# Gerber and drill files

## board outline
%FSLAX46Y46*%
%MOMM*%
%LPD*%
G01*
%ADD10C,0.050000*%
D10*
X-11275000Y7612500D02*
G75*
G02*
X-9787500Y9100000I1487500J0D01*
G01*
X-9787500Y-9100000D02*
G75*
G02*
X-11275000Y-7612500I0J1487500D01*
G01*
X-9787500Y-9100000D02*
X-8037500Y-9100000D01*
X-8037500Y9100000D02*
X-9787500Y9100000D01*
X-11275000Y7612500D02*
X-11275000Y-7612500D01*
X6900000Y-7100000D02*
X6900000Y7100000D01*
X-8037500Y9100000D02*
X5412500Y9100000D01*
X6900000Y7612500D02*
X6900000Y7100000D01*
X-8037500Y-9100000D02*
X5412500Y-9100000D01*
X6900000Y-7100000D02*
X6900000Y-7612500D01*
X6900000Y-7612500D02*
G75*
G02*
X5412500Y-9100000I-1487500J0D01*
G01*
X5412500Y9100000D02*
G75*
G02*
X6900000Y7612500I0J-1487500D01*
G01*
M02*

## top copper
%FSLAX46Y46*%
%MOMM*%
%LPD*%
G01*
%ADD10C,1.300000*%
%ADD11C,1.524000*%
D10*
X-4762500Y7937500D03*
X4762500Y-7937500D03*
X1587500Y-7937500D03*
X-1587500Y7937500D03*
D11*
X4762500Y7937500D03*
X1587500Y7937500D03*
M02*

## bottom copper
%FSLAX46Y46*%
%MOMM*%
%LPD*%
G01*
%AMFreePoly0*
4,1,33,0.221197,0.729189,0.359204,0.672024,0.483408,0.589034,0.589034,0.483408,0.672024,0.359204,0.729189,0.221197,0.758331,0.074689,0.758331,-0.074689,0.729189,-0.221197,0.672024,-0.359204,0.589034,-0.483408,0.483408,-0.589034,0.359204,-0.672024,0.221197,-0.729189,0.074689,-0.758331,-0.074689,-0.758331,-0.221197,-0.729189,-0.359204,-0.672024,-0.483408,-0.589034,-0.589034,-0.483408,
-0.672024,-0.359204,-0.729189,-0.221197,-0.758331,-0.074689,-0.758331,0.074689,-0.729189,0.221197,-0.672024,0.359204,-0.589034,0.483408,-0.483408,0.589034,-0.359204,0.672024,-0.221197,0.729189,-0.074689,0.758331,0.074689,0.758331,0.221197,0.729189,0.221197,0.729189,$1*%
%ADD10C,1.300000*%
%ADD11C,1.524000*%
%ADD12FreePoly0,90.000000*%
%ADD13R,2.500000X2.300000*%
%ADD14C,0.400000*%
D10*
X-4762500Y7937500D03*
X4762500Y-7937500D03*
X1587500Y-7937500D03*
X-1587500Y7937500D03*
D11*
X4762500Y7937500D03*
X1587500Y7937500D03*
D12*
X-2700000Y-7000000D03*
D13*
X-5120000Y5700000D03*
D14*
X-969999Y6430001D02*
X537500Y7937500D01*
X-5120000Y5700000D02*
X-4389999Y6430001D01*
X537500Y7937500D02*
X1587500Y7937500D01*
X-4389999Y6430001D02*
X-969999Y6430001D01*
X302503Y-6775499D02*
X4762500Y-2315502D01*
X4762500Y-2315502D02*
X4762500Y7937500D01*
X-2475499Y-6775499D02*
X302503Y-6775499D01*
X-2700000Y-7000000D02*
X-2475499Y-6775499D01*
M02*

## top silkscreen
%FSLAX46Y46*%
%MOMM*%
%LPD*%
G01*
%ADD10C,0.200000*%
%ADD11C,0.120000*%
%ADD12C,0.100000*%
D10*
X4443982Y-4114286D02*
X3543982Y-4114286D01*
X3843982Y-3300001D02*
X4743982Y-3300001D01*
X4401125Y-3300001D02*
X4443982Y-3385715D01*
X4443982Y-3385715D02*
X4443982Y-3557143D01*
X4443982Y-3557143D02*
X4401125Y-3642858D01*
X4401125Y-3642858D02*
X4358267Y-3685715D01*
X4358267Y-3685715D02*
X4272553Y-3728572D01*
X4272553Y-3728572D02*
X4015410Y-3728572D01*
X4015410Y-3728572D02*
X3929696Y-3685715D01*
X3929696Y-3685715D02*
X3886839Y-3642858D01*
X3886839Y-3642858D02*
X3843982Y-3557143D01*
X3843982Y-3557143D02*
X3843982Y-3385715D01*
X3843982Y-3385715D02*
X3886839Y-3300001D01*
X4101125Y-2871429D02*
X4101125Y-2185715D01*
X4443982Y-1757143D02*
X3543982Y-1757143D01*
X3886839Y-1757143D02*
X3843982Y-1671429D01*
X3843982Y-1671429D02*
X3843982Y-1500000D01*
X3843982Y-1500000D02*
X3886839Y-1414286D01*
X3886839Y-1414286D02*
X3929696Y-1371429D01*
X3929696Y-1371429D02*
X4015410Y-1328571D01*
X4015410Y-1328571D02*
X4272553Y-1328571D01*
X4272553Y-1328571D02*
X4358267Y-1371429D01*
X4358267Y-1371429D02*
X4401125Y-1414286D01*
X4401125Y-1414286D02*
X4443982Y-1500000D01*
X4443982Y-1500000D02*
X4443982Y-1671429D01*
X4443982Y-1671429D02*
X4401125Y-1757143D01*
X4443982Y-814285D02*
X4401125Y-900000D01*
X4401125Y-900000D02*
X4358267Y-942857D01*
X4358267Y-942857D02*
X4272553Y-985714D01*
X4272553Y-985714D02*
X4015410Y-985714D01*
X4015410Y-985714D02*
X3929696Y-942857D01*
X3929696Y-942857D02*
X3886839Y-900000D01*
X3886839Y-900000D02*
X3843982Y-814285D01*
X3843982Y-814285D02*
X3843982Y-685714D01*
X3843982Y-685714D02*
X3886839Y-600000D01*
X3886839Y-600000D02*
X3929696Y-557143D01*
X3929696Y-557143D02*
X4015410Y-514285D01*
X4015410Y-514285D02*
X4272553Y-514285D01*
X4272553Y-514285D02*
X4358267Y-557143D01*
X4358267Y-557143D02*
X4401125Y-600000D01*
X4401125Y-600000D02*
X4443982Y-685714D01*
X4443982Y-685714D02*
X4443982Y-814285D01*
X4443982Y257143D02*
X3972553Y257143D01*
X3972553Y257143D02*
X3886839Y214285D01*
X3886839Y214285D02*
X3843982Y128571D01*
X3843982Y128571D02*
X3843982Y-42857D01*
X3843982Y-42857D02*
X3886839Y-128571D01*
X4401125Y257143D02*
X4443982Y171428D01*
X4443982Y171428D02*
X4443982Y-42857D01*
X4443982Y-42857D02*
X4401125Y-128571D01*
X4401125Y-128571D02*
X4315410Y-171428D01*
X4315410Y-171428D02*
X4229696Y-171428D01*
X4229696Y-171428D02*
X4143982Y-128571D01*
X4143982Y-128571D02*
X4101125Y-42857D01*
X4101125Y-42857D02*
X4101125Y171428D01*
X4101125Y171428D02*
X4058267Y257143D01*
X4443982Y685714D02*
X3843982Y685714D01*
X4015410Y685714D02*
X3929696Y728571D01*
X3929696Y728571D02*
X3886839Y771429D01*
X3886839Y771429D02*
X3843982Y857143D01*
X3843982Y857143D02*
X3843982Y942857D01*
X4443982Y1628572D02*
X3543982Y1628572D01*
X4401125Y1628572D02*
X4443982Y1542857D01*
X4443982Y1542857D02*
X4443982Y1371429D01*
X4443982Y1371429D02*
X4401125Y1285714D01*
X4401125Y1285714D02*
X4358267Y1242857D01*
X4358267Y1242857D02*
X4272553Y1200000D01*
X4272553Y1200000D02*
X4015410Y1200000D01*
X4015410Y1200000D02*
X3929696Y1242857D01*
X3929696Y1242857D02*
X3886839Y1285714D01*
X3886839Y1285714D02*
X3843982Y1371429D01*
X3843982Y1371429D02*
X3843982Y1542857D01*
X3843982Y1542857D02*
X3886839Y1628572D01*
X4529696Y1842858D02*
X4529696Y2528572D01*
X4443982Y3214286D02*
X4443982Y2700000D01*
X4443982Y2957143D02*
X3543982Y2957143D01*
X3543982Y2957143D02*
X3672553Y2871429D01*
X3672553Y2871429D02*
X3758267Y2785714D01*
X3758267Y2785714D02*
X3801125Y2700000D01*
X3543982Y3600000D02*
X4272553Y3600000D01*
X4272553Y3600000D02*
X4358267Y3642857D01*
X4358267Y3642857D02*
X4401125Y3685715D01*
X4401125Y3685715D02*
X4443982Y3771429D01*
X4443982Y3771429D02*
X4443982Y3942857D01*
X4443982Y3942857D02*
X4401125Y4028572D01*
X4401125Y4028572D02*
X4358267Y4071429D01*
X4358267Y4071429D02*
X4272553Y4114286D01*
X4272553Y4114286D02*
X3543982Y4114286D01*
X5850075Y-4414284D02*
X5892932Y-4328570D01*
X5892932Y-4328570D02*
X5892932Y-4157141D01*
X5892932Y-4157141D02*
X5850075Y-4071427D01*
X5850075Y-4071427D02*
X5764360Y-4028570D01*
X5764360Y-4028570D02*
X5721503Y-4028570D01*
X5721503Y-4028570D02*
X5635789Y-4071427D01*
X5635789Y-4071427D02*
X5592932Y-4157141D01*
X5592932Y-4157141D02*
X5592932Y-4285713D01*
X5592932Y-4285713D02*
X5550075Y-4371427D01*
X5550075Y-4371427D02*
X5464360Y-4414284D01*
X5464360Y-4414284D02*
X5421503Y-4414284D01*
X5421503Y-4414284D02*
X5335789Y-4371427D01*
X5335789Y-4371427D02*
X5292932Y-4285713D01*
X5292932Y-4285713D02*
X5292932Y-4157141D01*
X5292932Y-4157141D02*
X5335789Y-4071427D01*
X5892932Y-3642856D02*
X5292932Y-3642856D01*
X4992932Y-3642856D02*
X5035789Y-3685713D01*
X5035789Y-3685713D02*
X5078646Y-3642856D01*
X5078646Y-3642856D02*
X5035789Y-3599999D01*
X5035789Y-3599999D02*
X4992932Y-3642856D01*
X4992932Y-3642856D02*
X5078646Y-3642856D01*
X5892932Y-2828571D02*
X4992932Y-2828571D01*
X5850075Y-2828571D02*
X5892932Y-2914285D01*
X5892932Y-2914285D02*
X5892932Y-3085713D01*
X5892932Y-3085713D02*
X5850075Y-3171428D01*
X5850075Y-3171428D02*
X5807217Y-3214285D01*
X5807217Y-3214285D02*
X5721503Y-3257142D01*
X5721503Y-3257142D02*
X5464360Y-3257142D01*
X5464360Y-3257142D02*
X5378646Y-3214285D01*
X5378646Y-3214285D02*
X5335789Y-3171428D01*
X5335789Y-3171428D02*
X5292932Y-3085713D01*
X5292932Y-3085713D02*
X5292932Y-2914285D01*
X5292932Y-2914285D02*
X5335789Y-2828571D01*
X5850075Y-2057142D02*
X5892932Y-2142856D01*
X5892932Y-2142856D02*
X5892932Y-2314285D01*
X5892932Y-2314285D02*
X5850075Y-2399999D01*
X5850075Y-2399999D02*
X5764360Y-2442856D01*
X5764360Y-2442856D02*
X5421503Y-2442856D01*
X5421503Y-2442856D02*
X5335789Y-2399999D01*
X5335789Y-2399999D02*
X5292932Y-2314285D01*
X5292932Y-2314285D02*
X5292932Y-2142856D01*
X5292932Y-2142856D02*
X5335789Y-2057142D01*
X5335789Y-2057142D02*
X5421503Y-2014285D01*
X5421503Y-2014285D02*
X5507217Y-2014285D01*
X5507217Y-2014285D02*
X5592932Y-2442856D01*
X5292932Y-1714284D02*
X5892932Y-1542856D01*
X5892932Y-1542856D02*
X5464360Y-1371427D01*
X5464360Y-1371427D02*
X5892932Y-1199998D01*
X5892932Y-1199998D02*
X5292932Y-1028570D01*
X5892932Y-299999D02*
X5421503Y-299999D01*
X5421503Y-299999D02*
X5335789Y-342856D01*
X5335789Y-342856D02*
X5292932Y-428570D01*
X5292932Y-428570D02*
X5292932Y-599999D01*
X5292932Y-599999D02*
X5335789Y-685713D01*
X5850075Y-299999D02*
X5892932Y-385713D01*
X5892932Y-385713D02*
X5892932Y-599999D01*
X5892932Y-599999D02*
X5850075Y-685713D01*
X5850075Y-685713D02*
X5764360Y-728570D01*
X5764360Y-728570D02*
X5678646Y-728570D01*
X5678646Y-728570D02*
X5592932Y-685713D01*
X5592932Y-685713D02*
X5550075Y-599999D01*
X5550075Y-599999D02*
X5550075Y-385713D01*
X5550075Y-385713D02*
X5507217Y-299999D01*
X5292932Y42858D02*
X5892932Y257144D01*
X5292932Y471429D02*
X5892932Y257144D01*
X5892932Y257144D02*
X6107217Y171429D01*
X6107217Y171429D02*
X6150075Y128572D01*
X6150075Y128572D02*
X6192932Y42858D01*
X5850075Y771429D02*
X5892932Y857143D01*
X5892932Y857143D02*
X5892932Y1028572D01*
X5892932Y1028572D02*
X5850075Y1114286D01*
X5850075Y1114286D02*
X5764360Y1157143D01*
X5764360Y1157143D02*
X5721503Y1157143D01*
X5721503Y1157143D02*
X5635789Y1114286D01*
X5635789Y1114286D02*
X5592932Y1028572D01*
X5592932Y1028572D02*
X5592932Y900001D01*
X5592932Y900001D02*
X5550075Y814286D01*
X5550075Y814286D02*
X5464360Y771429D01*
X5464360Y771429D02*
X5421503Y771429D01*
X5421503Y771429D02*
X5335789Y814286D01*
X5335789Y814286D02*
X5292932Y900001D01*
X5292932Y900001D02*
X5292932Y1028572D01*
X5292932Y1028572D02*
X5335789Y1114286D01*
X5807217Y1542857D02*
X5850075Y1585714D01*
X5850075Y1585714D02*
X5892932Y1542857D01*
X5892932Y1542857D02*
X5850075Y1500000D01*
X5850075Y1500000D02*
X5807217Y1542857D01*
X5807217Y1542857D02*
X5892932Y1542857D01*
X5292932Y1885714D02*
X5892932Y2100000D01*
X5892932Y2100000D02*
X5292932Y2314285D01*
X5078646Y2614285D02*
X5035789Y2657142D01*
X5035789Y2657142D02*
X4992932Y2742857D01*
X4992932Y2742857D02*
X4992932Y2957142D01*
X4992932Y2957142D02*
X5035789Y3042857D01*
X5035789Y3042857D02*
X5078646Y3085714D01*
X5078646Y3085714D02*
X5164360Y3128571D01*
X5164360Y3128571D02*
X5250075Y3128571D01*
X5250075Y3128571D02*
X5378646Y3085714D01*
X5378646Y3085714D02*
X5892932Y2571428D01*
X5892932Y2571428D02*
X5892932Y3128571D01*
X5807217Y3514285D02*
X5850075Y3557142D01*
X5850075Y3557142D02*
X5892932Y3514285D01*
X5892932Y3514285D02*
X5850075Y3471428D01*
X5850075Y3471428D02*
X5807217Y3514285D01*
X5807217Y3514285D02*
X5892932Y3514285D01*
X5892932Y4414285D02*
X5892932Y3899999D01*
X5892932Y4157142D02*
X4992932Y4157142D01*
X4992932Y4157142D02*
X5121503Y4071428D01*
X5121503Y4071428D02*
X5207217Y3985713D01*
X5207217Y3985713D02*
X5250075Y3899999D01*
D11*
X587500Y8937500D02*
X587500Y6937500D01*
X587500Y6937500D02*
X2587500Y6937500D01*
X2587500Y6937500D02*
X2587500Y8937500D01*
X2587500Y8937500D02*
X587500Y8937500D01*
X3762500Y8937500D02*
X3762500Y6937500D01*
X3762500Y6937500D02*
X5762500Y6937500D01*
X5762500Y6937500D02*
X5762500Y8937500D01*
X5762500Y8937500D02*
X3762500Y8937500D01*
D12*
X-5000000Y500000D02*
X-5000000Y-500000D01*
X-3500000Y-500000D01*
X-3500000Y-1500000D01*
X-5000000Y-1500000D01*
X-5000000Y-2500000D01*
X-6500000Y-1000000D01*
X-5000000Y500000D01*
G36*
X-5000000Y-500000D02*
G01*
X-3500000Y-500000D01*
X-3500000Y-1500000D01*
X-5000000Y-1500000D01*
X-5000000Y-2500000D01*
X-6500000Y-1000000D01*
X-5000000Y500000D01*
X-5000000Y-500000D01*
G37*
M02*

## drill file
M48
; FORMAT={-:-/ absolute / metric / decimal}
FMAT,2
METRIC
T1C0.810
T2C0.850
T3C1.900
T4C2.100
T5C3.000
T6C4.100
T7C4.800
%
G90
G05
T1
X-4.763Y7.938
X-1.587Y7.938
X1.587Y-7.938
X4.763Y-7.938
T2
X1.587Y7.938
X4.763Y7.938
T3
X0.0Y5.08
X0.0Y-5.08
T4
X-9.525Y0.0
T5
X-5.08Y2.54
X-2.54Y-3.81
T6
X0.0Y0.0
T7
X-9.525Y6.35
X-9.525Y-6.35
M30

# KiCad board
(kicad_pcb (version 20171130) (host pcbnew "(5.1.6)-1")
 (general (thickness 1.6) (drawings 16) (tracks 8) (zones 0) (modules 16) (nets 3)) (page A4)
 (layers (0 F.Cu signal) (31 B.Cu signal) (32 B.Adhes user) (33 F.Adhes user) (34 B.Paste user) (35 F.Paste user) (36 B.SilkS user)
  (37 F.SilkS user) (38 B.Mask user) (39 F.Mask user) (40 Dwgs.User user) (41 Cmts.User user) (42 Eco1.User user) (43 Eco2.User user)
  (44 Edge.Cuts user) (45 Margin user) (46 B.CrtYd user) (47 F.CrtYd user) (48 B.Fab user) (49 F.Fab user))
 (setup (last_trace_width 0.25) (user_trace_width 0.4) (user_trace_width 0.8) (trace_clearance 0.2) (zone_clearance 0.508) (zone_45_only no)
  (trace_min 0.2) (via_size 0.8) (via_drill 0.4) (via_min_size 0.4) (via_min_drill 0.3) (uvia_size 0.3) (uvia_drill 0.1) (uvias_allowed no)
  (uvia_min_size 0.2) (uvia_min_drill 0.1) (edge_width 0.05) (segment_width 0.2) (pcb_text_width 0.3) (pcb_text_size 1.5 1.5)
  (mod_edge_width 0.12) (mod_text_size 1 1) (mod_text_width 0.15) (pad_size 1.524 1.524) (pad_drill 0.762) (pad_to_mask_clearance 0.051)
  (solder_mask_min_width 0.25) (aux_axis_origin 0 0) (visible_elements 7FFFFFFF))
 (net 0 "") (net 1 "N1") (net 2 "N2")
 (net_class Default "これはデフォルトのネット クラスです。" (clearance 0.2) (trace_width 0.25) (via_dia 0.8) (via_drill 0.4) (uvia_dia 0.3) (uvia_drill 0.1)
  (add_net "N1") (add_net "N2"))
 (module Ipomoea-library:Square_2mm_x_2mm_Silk (layer F.Cu) (at 1.5875 -7.9375)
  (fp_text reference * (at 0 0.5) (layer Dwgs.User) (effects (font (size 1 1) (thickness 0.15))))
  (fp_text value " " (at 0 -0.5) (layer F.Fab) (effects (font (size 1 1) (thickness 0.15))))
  (fp_line (start -1 -1) (end -1 1) (layer F.SilkS) (width 0.12))
  (fp_line (start -1 1) (end 1 1) (layer F.SilkS) (width 0.12))
  (fp_line (start 1 1) (end 1 -1) (layer F.SilkS) (width 0.12))
  (fp_line (start 1 -1) (end -1 -1) (layer F.SilkS) (width 0.12)))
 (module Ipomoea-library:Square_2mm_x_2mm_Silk (layer F.Cu) (at 4.7625 -7.9375)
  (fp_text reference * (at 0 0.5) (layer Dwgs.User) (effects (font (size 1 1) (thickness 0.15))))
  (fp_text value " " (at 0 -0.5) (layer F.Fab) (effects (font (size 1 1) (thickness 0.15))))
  (fp_line (start -1 -1) (end -1 1) (layer F.SilkS) (width 0.12))
  (fp_line (start -1 1) (end 1 1) (layer F.SilkS) (width 0.12))
  (fp_line (start 1 1) (end 1 -1) (layer F.SilkS) (width 0.12))
  (fp_line (start 1 -1) (end -1 -1) (layer F.SilkS) (width 0.12)))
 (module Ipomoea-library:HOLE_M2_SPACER (layer F.Cu) (at -9.525 6.35)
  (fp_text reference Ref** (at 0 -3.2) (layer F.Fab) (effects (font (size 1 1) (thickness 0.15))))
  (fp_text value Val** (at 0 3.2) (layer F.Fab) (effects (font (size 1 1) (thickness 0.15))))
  (pad "" np_thru_hole circle (at 0 0) (size 4.8 4.8) (drill 4.8) (layers *.Cu *.Mask)))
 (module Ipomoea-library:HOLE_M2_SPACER (layer F.Cu) (at -9.525 -6.35)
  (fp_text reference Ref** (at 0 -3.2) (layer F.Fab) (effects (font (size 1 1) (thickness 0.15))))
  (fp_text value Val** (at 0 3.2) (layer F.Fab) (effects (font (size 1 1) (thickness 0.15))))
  (pad "" np_thru_hole circle (at 0 0) (size 4.8 4.8) (drill 4.8) (layers *.Cu *.Mask)))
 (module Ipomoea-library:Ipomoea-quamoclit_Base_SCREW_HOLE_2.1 (layer F.Cu) (at -9.525 0)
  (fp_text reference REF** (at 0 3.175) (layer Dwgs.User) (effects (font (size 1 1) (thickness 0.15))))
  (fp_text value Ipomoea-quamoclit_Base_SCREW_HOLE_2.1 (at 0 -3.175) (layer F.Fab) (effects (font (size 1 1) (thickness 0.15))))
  (pad "" np_thru_hole circle (at 0 0) (size 2.1 2.1) (drill 2.1) (layers *.Cu *.Mask)))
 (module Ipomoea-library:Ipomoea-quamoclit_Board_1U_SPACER (layer F.Cu) (at 0 0)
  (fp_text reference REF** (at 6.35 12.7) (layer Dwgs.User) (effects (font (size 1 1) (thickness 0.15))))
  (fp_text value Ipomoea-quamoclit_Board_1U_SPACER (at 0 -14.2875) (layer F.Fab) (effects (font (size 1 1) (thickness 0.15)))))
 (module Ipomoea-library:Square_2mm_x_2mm (layer F.Cu) (at 1.5875 7.9375)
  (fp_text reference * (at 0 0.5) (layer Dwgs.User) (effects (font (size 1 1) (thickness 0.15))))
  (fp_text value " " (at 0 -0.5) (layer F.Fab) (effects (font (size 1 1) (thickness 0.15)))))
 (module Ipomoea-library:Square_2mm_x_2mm (layer F.Cu) (at 4.7625 7.9375)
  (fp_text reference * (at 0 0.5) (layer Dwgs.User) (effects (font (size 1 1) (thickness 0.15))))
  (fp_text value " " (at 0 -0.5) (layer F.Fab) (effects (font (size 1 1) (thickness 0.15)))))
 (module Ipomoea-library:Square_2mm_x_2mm (layer F.Cu) (at -4.7625 -7.9375)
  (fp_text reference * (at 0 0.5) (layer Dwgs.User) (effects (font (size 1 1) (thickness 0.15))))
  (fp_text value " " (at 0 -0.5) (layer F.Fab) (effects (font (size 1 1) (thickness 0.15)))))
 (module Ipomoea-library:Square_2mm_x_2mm (layer F.Cu) (at -1.5875 -7.9375)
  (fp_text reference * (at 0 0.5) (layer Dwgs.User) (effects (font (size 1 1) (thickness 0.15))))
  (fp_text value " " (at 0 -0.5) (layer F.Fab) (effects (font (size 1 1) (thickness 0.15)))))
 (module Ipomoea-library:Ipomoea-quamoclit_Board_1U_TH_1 (layer F.Cu) (at -4.7625 -7.9375)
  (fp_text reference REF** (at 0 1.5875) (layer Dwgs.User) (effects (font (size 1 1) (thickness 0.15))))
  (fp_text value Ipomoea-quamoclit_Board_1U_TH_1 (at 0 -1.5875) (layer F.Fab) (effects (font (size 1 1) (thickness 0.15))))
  (pad "" thru_hole circle (at 0 0 180) (size 1.3 1.3) (drill 0.81) (layers *.Cu *.Mask)))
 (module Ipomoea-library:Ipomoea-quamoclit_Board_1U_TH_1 (layer F.Cu) (at 4.7625 7.9375)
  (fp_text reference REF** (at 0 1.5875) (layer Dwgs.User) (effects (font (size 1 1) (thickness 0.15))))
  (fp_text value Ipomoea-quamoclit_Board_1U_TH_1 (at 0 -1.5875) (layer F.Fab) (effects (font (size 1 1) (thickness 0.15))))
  (pad "" thru_hole circle (at 0 0 180) (size 1.3 1.3) (drill 0.81) (layers *.Cu *.Mask)))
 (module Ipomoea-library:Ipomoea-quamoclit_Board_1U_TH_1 (layer F.Cu) (at 1.5875 7.9375)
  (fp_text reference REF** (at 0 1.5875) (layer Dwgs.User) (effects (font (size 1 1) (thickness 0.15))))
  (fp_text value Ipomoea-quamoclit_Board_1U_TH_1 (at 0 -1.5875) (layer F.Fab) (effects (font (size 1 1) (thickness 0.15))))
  (pad "" thru_hole circle (at 0 0 180) (size 1.3 1.3) (drill 0.81) (layers *.Cu *.Mask)))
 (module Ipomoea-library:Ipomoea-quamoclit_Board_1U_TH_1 (layer F.Cu) (at -1.5875 -7.9375)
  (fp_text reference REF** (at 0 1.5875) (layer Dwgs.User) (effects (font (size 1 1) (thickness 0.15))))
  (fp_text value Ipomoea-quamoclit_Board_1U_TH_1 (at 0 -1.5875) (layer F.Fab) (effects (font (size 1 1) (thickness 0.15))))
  (pad "" thru_hole circle (at 0 0 180) (size 1.3 1.3) (drill 0.81) (layers *.Cu *.Mask)))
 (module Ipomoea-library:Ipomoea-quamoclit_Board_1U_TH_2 (layer F.Cu) (at 3.175 -7.9375 180)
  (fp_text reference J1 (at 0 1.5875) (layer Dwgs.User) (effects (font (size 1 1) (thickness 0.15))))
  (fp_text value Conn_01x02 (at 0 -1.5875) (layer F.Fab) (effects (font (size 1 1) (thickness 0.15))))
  (pad 1 thru_hole circle (at -1.5875 0) (size 1.524 1.524) (drill 0.85) (layers *.Cu *.Mask) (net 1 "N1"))
  (pad 2 thru_hole circle (at 1.5875 0) (size 1.524 1.524) (drill 0.85) (layers *.Cu *.Mask) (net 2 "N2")))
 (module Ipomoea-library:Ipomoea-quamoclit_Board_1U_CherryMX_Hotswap (layer F.Cu) (at 0 0 90)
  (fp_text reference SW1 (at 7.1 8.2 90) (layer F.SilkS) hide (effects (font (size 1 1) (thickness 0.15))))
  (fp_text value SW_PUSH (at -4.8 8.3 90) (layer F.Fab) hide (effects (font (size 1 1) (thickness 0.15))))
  (fp_poly (pts (xy 0.5 -5) (xy -0.5 -5) (xy -0.5 -3.5) (xy -1.5 -3.5) (xy -1.5 -5) (xy -2.5 -5) (xy -1 -6.5)) (layer F.SilkS) (width 0.1))
  (pad "" np_thru_hole circle (at 0 0 180) (size 4.1 4.1) (drill 4.1) (layers *.Cu *.Mask))
  (pad "" np_thru_hole circle (at 5.08 0 90) (size 1.9 1.9) (drill 1.9) (layers *.Cu *.Mask))
  (pad "" np_thru_hole circle (at -5.08 0 90) (size 1.9 1.9) (drill 1.9) (layers *.Cu *.Mask))
  (pad 1 smd custom (at -7 -2.7 90) (size 1.524 1.524) (layers B.Cu B.Paste B.Mask) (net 1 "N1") (zone_connect 0)
   (options (clearance outline) (anchor circle)) (primitives))
  (pad "" np_thru_hole circle (at 2.54 -5.08 270) (size 3 3) (drill 3) (layers *.Cu *.Mask))
  (pad 2 smd rect (at 5.7 -5.12 270) (size 2.3 2.5) (layers B.Cu B.Paste B.Mask) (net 2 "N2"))
  (pad "" np_thru_hole circle (at -3.81 -2.54 270) (size 3 3) (drill 3) (layers *.Cu *.Mask)))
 (gr_arc (start -9.7875 -7.6125) (end -9.7875 -9.1) (angle -90) (layer Edge.Cuts) (width 0.05))
 (gr_arc (start -9.7875 7.6125) (end -11.275 7.6125) (angle -90) (layer Edge.Cuts) (width 0.05))
 (gr_line (start -9.7875 9.1) (end -8.0375 9.1) (layer Edge.Cuts) (width 0.05))
 (gr_line (start -8.0375 -9.1) (end -9.7875 -9.1) (layer Edge.Cuts) (width 0.05))
 (gr_line (start -11.275 -7.6125) (end -11.275 7.6125) (layer Edge.Cuts) (width 0.05))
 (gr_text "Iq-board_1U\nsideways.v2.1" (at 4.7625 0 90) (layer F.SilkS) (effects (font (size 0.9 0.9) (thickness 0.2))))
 (gr_line (start 6.9 7.1) (end 6.9 -7.1) (layer Edge.Cuts) (width 0.05))
 (gr_line (start -8.0375 -9.1) (end 5.4125 -9.1) (layer Edge.Cuts) (width 0.05))
 (gr_line (start 6.9 -7.6125) (end 6.9 -7.1) (layer Edge.Cuts) (width 0.05))
 (gr_line (start -8.0375 9.1) (end 5.4125 9.1) (layer Edge.Cuts) (width 0.05))
 (gr_line (start 6.9 7.1) (end 6.9 7.6125) (layer Edge.Cuts) (width 0.05))
 (gr_arc (start 5.4125 7.6125) (end 5.4125 9.1) (angle -90) (layer Edge.Cuts) (width 0.05))
 (gr_arc (start 5.4125 -7.6125) (end 6.9 -7.6125) (angle -90) (layer Edge.Cuts) (width 0.05))
 (segment (start -0.969999 -6.430001) (end 0.5375 -7.9375) (width 0.4) (layer B.Cu) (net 2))
 (segment (start -5.12 -5.7) (end -4.389999 -6.430001) (width 0.4) (layer B.Cu) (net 2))
 (segment (start 0.5375 -7.9375) (end 1.5875 -7.9375) (width 0.4) (layer B.Cu) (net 2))
 (segment (start -4.389999 -6.430001) (end -0.969999 -6.430001) (width 0.4) (layer B.Cu) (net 2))
 (segment (start 0.302503 6.775499) (end 4.7625 2.315502) (width 0.4) (layer B.Cu) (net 1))
 (segment (start 4.7625 2.315502) (end 4.7625 -7.9375) (width 0.4) (layer B.Cu) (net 1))
 (segment (start -2.475499 6.775499) (end 0.302503 6.775499) (width 0.4) (layer B.Cu) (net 1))
 (segment (start -2.7 7) (end -2.475499 6.775499) (width 0.4) (layer B.Cu) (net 1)))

